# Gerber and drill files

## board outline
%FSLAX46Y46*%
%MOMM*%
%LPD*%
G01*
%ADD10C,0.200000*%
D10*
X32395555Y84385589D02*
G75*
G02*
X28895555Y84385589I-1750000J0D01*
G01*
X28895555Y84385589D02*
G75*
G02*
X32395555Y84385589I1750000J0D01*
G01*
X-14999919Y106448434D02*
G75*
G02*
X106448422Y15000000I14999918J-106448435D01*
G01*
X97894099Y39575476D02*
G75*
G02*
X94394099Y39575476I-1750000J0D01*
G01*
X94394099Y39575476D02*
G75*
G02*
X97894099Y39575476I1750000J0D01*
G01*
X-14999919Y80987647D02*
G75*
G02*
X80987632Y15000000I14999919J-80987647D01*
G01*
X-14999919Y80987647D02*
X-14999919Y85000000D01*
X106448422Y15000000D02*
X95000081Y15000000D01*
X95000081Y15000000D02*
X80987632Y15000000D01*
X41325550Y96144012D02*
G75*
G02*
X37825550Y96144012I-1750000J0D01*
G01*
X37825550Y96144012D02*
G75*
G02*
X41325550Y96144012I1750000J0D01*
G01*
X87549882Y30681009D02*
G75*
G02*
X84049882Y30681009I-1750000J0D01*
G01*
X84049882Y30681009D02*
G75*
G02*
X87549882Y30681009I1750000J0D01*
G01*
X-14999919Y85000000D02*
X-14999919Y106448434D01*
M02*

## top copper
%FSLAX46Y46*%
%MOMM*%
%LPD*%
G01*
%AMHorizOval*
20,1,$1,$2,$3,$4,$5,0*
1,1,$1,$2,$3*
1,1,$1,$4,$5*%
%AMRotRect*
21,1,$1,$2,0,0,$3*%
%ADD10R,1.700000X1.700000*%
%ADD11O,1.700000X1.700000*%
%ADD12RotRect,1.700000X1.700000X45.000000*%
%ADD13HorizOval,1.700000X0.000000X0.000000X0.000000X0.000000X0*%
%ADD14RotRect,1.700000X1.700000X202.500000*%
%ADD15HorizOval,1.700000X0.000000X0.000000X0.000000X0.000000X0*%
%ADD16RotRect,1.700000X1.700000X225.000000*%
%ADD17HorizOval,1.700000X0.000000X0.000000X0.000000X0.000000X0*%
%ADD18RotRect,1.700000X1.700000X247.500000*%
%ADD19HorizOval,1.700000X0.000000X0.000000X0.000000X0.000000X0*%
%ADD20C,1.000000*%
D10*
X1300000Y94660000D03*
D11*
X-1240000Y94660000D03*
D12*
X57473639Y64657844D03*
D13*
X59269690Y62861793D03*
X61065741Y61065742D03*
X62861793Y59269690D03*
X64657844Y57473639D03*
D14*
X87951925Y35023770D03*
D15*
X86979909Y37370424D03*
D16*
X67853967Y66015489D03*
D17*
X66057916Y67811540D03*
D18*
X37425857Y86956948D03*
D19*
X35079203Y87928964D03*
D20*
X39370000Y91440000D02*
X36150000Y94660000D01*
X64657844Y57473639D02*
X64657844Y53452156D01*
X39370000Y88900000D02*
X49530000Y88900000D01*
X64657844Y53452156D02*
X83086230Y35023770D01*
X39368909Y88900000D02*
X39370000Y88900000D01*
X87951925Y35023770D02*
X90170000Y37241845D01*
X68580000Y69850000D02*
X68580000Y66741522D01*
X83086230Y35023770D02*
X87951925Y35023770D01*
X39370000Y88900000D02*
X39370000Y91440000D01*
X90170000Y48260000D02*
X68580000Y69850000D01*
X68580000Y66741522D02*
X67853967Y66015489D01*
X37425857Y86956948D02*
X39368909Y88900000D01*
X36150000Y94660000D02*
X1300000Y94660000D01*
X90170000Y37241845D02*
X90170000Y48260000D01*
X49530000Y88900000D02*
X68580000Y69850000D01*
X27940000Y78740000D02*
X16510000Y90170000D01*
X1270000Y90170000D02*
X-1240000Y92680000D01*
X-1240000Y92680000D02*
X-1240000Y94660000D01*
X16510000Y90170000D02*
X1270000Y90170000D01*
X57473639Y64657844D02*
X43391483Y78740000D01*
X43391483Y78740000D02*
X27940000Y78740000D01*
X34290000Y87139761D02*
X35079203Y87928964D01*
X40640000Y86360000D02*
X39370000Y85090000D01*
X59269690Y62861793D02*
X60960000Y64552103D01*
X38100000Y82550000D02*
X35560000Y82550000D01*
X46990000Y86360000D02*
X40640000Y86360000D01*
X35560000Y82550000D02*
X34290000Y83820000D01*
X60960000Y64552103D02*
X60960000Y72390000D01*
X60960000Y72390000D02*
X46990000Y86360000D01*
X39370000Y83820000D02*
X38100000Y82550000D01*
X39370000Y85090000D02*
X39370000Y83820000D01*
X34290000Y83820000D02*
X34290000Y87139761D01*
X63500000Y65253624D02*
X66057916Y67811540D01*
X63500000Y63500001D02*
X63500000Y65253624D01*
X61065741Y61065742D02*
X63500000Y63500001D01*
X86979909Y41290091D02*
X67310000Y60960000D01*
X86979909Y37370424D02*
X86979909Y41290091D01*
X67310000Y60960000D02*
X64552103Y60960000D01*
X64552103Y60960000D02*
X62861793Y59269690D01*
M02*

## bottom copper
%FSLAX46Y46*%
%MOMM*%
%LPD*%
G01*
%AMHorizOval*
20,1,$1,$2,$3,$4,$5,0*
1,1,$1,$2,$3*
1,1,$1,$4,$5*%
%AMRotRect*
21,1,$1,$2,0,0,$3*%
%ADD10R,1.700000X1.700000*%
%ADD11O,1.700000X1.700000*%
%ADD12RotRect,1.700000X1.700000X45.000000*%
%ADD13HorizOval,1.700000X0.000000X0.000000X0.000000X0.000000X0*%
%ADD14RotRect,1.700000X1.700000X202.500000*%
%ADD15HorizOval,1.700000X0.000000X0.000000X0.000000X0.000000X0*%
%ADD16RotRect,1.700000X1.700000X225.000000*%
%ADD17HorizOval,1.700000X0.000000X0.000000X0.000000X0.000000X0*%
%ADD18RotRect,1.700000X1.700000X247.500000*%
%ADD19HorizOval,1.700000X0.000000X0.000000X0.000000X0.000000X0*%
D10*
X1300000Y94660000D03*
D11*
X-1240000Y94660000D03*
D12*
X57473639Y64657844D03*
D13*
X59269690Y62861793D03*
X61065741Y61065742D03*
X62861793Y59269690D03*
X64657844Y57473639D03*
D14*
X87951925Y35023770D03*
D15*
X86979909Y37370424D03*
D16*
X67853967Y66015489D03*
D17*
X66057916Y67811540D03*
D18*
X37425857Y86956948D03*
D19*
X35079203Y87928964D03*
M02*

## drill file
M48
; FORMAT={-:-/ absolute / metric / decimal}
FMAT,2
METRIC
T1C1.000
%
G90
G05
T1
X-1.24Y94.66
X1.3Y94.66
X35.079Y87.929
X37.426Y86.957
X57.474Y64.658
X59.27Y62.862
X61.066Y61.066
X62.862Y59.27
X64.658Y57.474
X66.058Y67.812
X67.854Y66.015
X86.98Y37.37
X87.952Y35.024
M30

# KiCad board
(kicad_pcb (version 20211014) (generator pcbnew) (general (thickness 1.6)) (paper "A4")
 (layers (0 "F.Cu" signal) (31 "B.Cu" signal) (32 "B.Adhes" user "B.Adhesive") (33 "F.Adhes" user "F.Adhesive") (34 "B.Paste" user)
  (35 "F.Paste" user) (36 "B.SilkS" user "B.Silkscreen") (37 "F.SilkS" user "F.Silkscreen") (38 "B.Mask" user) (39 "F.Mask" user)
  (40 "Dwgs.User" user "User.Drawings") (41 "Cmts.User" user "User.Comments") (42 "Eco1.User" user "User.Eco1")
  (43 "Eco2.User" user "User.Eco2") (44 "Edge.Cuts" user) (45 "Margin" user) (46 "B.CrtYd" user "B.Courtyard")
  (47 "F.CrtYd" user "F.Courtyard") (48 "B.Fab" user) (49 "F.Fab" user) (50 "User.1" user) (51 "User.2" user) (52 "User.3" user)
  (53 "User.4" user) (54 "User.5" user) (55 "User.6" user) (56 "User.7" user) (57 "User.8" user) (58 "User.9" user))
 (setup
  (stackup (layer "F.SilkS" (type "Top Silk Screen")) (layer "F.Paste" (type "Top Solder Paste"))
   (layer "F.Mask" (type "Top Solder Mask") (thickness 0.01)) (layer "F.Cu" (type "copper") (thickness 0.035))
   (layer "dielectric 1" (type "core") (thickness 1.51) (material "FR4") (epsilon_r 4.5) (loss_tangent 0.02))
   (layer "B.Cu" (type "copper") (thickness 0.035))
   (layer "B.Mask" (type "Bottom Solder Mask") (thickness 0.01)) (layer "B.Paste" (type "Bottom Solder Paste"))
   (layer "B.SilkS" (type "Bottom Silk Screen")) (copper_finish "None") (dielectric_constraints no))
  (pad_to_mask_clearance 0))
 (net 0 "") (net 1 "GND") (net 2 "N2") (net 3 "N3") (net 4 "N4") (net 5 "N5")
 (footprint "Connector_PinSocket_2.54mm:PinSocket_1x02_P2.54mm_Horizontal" (layer "F.Cu") (at 1.3 -94.66 -90)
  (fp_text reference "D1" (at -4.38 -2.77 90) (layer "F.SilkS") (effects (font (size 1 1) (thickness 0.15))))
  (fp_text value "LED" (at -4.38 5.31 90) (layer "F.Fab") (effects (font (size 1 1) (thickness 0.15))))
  (pad "1" thru_hole rect (at 0 0 270) (size 1.7 1.7) (drill 1) (layers *.Cu *.Mask) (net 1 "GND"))
  (pad "2" thru_hole oval (at 0 2.54 270) (size 1.7 1.7) (drill 1) (layers *.Cu *.Mask) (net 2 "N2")))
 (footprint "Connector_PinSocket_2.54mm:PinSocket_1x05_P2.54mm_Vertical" (layer "F.Cu") (at 57.473639 -64.657844 45)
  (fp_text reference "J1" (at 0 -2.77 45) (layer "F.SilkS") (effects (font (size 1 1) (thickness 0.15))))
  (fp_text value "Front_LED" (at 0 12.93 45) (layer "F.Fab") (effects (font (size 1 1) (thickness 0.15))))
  (pad "1" thru_hole rect (at 0 0 45) (size 1.7 1.7) (drill 1) (layers *.Cu *.Mask) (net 2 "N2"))
  (pad "2" thru_hole oval (at 0 2.54 45) (size 1.7 1.7) (drill 1) (layers *.Cu *.Mask) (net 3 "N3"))
  (pad "3" thru_hole oval (at 0 5.08 45) (size 1.7 1.7) (drill 1) (layers *.Cu *.Mask) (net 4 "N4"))
  (pad "4" thru_hole oval (at 0 7.62 45) (size 1.7 1.7) (drill 1) (layers *.Cu *.Mask) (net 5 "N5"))
  (pad "5" thru_hole oval (at 0 10.16 45) (size 1.7 1.7) (drill 1) (layers *.Cu *.Mask) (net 1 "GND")))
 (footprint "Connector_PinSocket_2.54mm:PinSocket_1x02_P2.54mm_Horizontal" (layer "F.Cu") (at 87.951925 -35.02377 -157.5)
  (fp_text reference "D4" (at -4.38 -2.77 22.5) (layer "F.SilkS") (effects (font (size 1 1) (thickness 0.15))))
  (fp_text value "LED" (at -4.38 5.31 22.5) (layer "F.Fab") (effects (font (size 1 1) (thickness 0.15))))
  (pad "1" thru_hole rect (at 0 0 202.5) (size 1.7 1.7) (drill 1) (layers *.Cu *.Mask) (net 1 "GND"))
  (pad "2" thru_hole oval (at 0 2.54 202.5) (size 1.7 1.7) (drill 1) (layers *.Cu *.Mask) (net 5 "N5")))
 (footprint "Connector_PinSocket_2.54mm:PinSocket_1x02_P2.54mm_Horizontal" (layer "F.Cu") (at 67.853967 -66.015489 -135)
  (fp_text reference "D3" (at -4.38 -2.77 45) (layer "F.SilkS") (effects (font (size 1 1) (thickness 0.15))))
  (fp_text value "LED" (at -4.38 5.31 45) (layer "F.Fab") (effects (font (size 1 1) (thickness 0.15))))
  (pad "1" thru_hole rect (at 0 0 225) (size 1.7 1.7) (drill 1) (layers *.Cu *.Mask) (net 1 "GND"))
  (pad "2" thru_hole oval (at 0 2.54 225) (size 1.7 1.7) (drill 1) (layers *.Cu *.Mask) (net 4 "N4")))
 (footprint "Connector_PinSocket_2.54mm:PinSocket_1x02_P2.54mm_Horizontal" (layer "F.Cu") (at 37.425857 -86.956948 -112.5)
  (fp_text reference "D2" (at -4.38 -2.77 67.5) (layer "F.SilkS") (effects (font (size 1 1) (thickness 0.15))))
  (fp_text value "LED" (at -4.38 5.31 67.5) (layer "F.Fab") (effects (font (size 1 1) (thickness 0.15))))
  (pad "1" thru_hole rect (at 0 0 247.5) (size 1.7 1.7) (drill 1) (layers *.Cu *.Mask) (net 1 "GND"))
  (pad "2" thru_hole oval (at 0 2.54 247.5) (size 1.7 1.7) (drill 1) (layers *.Cu *.Mask) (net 3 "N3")))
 (gr_circle (center 30.645555 -84.385589) (end 32.395555 -84.385589) (layer "Edge.Cuts") (width 0.2) (fill none))
 (gr_arc (start -14.999919 -106.448434) (mid 64.663832 -85.876978) (end 106.448422 -15) (layer "Edge.Cuts") (width 0.2))
 (gr_circle (center 96.144099 -39.575476) (end 97.894099 -39.575476) (layer "Edge.Cuts") (width 0.2) (fill none))
 (gr_arc (start -14.999919 -80.987647) (mid 46.660336 -67.873482) (end 80.987632 -15) (layer "Edge.Cuts") (width 0.2))
 (gr_line (start -14.999919 -80.987647) (end -14.999919 -85) (layer "Edge.Cuts") (width 0.2))
 (gr_line (start 106.448422 -15) (end 95.000081 -15) (layer "Edge.Cuts") (width 0.2))
 (gr_line (start 95.000081 -15) (end 80.987632 -15) (layer "Edge.Cuts") (width 0.2))
 (gr_circle (center 39.57555 -96.144012) (end 41.32555 -96.144012) (layer "Edge.Cuts") (width 0.2) (fill none))
 (gr_circle (center 85.799882 -30.681009) (end 87.549882 -30.681009) (layer "Edge.Cuts") (width 0.2) (fill none))
 (gr_line (start -14.999919 -85) (end -14.999919 -106.448434) (layer "Edge.Cuts") (width 0.2))
 (segment (start 39.37 -91.44) (end 36.15 -94.66) (width 1) (layer "F.Cu") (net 1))
 (segment (start 64.657844 -57.473639) (end 64.657844 -53.452156) (width 1) (layer "F.Cu") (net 1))
 (segment (start 39.37 -88.9) (end 49.53 -88.9) (width 1) (layer "F.Cu") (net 1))
 (segment (start 64.657844 -53.452156) (end 83.08623 -35.02377) (width 1) (layer "F.Cu") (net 1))
 (segment (start 39.368909 -88.9) (end 39.37 -88.9) (width 1) (layer "F.Cu") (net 1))
 (segment (start 87.951925 -35.02377) (end 90.17 -37.241845) (width 1) (layer "F.Cu") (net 1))
 (segment (start 68.58 -69.85) (end 68.58 -66.741522) (width 1) (layer "F.Cu") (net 1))
 (segment (start 83.08623 -35.02377) (end 87.951925 -35.02377) (width 1) (layer "F.Cu") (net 1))
 (segment (start 39.37 -88.9) (end 39.37 -91.44) (width 1) (layer "F.Cu") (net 1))
 (segment (start 90.17 -48.26) (end 68.58 -69.85) (width 1) (layer "F.Cu") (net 1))
 (segment (start 68.58 -66.741522) (end 67.853967 -66.015489) (width 1) (layer "F.Cu") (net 1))
 (segment (start 37.425857 -86.956948) (end 39.368909 -88.9) (width 1) (layer "F.Cu") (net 1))
 (segment (start 36.15 -94.66) (end 1.3 -94.66) (width 1) (layer "F.Cu") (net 1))
 (segment (start 90.17 -37.241845) (end 90.17 -48.26) (width 1) (layer "F.Cu") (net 1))
 (segment (start 49.53 -88.9) (end 68.58 -69.85) (width 1) (layer "F.Cu") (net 1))
 (segment (start 27.94 -78.74) (end 16.51 -90.17) (width 1) (layer "F.Cu") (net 2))
 (segment (start 1.27 -90.17) (end -1.24 -92.68) (width 1) (layer "F.Cu") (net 2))
 (segment (start -1.24 -92.68) (end -1.24 -94.66) (width 1) (layer "F.Cu") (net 2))
 (segment (start 16.51 -90.17) (end 1.27 -90.17) (width 1) (layer "F.Cu") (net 2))
 (segment (start 57.473639 -64.657844) (end 43.391483 -78.74) (width 1) (layer "F.Cu") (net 2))
 (segment (start 43.391483 -78.74) (end 27.94 -78.74) (width 1) (layer "F.Cu") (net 2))
 (segment (start 34.29 -87.139761) (end 35.079203 -87.928964) (width 1) (layer "F.Cu") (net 3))
 (segment (start 40.64 -86.36) (end 39.37 -85.09) (width 1) (layer "F.Cu") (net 3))
 (segment (start 59.26969 -62.861793) (end 60.96 -64.552103) (width 1) (layer "F.Cu") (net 3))
 (segment (start 38.1 -82.55) (end 35.56 -82.55) (width 1) (layer "F.Cu") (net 3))
 (segment (start 46.99 -86.36) (end 40.64 -86.36) (width 1) (layer "F.Cu") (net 3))
 (segment (start 35.56 -82.55) (end 34.29 -83.82) (width 1) (layer "F.Cu") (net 3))
 (segment (start 60.96 -64.552103) (end 60.96 -72.39) (width 1) (layer "F.Cu") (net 3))
 (segment (start 60.96 -72.39) (end 46.99 -86.36) (width 1) (layer "F.Cu") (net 3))
 (segment (start 39.37 -83.82) (end 38.1 -82.55) (width 1) (layer "F.Cu") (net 3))
 (segment (start 39.37 -85.09) (end 39.37 -83.82) (width 1) (layer "F.Cu") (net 3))
 (segment (start 34.29 -83.82) (end 34.29 -87.139761) (width 1) (layer "F.Cu") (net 3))
 (segment (start 63.5 -65.253624) (end 66.057916 -67.81154) (width 1) (layer "F.Cu") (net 4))
 (segment (start 63.5 -63.500001) (end 63.5 -65.253624) (width 1) (layer "F.Cu") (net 4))
 (segment (start 61.065741 -61.065742) (end 63.5 -63.500001) (width 1) (layer "F.Cu") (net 4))
 (segment (start 86.979909 -41.290091) (end 67.31 -60.96) (width 1) (layer "F.Cu") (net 5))
 (segment (start 86.979909 -37.370424) (end 86.979909 -41.290091) (width 1) (layer "F.Cu") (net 5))
 (segment (start 67.31 -60.96) (end 64.552103 -60.96) (width 1) (layer "F.Cu") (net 5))
 (segment (start 64.552103 -60.96) (end 62.861793 -59.26969) (width 1) (layer "F.Cu") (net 5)))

